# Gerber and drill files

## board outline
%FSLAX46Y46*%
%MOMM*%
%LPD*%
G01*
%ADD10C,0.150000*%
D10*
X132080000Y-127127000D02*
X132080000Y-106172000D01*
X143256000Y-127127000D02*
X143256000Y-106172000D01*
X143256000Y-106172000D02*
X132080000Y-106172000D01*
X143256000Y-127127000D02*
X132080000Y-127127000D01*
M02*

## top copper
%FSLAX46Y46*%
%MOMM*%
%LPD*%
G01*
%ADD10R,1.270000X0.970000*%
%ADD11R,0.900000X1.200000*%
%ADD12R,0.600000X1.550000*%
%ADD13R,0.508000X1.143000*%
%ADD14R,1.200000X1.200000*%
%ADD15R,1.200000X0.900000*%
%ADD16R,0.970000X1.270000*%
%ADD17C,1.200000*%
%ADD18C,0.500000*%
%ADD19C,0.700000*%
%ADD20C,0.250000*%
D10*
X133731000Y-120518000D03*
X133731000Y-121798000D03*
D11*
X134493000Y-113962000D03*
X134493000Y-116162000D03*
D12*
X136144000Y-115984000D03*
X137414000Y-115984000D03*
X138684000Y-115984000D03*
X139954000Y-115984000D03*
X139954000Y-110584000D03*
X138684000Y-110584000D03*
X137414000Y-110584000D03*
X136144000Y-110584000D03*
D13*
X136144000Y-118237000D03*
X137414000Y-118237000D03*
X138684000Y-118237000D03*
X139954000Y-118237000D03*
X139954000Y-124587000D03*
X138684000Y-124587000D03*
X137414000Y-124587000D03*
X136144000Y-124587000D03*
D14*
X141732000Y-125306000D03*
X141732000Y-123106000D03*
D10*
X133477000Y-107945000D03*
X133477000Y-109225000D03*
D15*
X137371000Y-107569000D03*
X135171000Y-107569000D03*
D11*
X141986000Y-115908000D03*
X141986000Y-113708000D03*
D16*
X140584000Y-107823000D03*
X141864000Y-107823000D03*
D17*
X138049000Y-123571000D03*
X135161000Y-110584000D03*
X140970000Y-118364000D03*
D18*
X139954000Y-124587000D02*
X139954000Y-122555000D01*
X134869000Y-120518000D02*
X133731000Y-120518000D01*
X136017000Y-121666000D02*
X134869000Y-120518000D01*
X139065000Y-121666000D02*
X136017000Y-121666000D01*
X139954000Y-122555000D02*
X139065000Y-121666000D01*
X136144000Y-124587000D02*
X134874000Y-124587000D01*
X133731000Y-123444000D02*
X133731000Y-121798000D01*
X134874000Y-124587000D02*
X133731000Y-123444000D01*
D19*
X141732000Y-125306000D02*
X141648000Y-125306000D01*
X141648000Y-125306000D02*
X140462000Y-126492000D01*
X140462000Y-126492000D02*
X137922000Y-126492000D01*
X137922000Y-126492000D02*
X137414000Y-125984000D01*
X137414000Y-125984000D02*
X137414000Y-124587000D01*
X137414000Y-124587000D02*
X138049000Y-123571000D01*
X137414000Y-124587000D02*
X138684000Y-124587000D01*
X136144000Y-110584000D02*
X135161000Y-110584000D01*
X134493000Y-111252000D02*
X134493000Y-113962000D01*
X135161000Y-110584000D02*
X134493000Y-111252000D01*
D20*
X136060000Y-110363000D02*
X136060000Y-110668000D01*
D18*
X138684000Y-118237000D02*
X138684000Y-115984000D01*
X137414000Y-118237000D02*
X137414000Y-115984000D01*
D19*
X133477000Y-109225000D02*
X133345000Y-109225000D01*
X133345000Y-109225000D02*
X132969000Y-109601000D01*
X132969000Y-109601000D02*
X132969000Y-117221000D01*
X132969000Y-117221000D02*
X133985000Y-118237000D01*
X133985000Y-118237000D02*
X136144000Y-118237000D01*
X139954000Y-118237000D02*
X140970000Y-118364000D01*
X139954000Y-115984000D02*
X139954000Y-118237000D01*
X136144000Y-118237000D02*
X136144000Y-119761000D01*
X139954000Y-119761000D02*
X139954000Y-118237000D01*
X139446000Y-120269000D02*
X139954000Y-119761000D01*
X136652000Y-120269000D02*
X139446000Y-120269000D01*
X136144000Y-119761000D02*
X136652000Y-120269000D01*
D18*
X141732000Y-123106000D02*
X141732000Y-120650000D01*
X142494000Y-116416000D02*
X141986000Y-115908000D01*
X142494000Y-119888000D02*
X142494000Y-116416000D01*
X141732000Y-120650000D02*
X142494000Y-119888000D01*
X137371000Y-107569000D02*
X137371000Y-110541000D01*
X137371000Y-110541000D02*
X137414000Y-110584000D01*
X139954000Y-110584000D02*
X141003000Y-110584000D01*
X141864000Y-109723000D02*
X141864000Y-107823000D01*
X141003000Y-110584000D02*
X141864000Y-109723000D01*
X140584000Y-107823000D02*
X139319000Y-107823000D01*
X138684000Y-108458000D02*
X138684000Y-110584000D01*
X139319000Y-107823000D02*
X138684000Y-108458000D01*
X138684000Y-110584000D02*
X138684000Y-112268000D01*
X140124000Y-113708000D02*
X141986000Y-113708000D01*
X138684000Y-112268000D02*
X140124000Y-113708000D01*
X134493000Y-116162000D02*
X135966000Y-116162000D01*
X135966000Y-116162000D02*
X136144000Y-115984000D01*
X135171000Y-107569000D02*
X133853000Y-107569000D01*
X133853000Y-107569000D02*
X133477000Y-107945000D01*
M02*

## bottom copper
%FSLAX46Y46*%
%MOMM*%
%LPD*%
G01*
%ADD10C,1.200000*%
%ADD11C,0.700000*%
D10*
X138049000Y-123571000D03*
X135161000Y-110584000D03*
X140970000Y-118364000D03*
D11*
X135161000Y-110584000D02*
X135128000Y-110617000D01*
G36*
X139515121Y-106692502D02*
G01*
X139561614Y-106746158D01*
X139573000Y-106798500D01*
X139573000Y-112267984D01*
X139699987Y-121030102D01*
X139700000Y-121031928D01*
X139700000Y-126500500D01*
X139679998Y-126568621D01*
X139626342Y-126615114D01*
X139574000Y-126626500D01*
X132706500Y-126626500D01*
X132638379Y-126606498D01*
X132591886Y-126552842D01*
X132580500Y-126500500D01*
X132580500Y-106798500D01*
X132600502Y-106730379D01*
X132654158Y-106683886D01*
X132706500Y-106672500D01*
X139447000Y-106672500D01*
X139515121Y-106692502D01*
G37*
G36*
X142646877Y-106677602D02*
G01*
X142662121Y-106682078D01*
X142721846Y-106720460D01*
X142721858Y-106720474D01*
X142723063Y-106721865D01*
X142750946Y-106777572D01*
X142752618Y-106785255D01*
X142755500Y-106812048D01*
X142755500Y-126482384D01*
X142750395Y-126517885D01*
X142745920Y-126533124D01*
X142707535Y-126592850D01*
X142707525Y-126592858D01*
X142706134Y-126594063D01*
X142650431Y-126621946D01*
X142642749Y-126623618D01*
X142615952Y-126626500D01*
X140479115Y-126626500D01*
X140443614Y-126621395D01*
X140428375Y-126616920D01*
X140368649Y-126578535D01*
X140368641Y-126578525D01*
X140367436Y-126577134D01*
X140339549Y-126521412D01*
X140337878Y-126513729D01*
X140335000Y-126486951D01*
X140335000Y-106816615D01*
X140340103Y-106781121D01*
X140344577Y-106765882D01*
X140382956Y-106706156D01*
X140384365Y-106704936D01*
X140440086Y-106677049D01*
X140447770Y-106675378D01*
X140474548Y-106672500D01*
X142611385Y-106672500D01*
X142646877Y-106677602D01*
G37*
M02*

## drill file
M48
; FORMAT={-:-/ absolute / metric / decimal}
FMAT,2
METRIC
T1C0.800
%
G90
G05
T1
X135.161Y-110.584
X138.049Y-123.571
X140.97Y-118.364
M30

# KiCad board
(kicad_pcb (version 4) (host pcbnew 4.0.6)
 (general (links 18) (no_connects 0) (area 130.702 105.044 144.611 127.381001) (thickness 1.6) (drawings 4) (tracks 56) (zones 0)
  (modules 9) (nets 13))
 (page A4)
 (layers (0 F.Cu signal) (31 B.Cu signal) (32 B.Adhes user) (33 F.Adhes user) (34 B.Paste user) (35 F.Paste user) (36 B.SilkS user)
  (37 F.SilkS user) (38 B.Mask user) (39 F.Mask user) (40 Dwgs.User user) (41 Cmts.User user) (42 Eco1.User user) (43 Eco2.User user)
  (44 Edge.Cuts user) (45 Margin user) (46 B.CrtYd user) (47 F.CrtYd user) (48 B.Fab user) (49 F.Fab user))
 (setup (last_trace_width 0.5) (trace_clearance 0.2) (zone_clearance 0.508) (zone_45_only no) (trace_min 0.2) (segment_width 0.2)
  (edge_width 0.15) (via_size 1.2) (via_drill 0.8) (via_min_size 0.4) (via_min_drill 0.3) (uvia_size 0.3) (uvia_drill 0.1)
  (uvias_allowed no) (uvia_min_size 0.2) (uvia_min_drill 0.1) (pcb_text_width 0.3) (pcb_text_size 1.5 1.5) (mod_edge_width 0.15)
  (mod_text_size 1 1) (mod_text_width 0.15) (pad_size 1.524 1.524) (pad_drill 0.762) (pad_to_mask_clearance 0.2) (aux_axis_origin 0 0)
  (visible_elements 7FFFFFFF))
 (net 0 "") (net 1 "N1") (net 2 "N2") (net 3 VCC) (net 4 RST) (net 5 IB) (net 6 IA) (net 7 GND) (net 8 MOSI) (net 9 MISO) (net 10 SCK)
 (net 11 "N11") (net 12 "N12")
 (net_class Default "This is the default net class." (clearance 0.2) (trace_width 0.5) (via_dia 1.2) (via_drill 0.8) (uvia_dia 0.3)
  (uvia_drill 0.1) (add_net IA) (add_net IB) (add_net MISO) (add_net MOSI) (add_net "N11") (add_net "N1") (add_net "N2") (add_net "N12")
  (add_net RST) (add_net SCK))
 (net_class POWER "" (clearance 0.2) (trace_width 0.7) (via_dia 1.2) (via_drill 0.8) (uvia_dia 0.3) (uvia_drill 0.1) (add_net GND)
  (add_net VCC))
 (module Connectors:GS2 (layer F.Cu) (at 133.731 121.158)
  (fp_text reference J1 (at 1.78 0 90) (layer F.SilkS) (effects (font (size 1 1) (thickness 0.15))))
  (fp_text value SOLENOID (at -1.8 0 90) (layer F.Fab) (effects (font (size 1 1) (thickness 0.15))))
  (pad 1 smd rect (at 0 -0.64) (size 1.27 0.97) (layers F.Cu F.Paste F.Mask) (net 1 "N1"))
  (pad 2 smd rect (at 0 0.64) (size 1.27 0.97) (layers F.Cu F.Paste F.Mask) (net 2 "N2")))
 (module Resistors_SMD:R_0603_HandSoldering (layer F.Cu) (at 134.493 115.062 270)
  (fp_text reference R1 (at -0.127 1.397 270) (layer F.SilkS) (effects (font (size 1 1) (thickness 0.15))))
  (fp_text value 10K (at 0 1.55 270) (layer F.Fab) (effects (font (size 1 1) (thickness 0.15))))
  (pad 1 smd rect (at -1.1 0 270) (size 1.2 0.9) (layers F.Cu F.Paste F.Mask) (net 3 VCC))
  (pad 2 smd rect (at 1.1 0 270) (size 1.2 0.9) (layers F.Cu F.Paste F.Mask) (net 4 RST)))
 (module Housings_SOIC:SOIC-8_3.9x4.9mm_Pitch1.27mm (layer F.Cu) (at 138.049 113.284 90)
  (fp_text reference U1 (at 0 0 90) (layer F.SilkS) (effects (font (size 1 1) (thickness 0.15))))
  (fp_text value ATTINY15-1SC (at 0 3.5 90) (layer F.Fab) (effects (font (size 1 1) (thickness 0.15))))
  (pad 1 smd rect (at -2.7 -1.905 90) (size 1.55 0.6) (layers F.Cu F.Paste F.Mask) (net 4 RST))
  (pad 2 smd rect (at -2.7 -0.635 90) (size 1.55 0.6) (layers F.Cu F.Paste F.Mask) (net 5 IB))
  (pad 3 smd rect (at -2.7 0.635 90) (size 1.55 0.6) (layers F.Cu F.Paste F.Mask) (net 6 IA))
  (pad 4 smd rect (at -2.7 1.905 90) (size 1.55 0.6) (layers F.Cu F.Paste F.Mask) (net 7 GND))
  (pad 5 smd rect (at 2.7 1.905 90) (size 1.55 0.6) (layers F.Cu F.Paste F.Mask) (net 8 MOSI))
  (pad 6 smd rect (at 2.7 0.635 90) (size 1.55 0.6) (layers F.Cu F.Paste F.Mask) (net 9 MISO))
  (pad 7 smd rect (at 2.7 -0.635 90) (size 1.55 0.6) (layers F.Cu F.Paste F.Mask) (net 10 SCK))
  (pad 8 smd rect (at 2.7 -1.905 90) (size 1.55 0.6) (layers F.Cu F.Paste F.Mask) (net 3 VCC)))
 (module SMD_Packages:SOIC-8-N (layer F.Cu) (at 138.049 121.412)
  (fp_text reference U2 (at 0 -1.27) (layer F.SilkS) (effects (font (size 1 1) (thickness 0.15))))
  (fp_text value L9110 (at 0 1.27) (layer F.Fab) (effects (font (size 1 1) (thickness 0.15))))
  (pad 8 smd rect (at -1.905 -3.175) (size 0.508 1.143) (layers F.Cu F.Paste F.Mask) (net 7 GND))
  (pad 7 smd rect (at -0.635 -3.175) (size 0.508 1.143) (layers F.Cu F.Paste F.Mask) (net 5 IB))
  (pad 6 smd rect (at 0.635 -3.175) (size 0.508 1.143) (layers F.Cu F.Paste F.Mask) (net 6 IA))
  (pad 5 smd rect (at 1.905 -3.175) (size 0.508 1.143) (layers F.Cu F.Paste F.Mask) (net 7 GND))
  (pad 4 smd rect (at 1.905 3.175) (size 0.508 1.143) (layers F.Cu F.Paste F.Mask) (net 1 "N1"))
  (pad 3 smd rect (at 0.635 3.175) (size 0.508 1.143) (layers F.Cu F.Paste F.Mask) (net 3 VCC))
  (pad 2 smd rect (at -0.635 3.175) (size 0.508 1.143) (layers F.Cu F.Paste F.Mask) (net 3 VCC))
  (pad 1 smd rect (at -1.905 3.175) (size 0.508 1.143) (layers F.Cu F.Paste F.Mask) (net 2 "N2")))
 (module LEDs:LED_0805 (layer F.Cu) (at 141.732 124.206 270)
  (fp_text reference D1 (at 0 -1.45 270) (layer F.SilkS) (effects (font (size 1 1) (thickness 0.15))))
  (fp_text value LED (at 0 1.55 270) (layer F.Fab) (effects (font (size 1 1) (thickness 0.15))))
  (pad 2 smd rect (at 1.1 0 90) (size 1.2 1.2) (layers F.Cu F.Paste F.Mask) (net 3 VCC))
  (pad 1 smd rect (at -1.1 0 90) (size 1.2 1.2) (layers F.Cu F.Paste F.Mask) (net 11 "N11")))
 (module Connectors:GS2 (layer F.Cu) (at 133.477 108.585)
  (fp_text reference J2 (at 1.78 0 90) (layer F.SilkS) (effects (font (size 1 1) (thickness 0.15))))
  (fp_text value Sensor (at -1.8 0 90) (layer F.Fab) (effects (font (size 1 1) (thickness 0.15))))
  (pad 1 smd rect (at 0 -0.64) (size 1.27 0.97) (layers F.Cu F.Paste F.Mask) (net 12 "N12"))
  (pad 2 smd rect (at 0 0.64) (size 1.27 0.97) (layers F.Cu F.Paste F.Mask) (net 7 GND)))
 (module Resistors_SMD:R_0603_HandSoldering (layer F.Cu) (at 136.271 107.569 180)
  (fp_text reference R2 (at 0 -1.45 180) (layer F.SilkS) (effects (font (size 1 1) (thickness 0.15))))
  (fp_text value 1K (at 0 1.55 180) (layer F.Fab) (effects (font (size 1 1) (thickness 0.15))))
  (pad 1 smd rect (at -1.1 0 180) (size 1.2 0.9) (layers F.Cu F.Paste F.Mask) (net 10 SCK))
  (pad 2 smd rect (at 1.1 0 180) (size 1.2 0.9) (layers F.Cu F.Paste F.Mask) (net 12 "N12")))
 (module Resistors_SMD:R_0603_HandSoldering (layer F.Cu) (at 141.986 114.808 90)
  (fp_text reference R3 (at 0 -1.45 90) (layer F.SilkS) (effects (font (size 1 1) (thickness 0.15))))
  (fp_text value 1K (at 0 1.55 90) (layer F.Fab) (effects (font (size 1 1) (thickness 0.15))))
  (pad 1 smd rect (at -1.1 0 90) (size 1.2 0.9) (layers F.Cu F.Paste F.Mask) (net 11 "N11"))
  (pad 2 smd rect (at 1.1 0 90) (size 1.2 0.9) (layers F.Cu F.Paste F.Mask) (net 9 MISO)))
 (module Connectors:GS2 (layer F.Cu) (at 141.224 107.823 90)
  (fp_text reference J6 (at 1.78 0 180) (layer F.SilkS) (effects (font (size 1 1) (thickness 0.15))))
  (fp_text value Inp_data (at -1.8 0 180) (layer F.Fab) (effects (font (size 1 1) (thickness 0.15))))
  (pad 1 smd rect (at 0 -0.64 90) (size 1.27 0.97) (layers F.Cu F.Paste F.Mask) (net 9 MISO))
  (pad 2 smd rect (at 0 0.64 90) (size 1.27 0.97) (layers F.Cu F.Paste F.Mask) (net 8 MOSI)))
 (gr_line (start 132.08 127.127) (end 132.08 106.172) (angle 90) (layer Edge.Cuts) (width 0.15))
 (gr_line (start 143.256 127.127) (end 143.256 106.172) (angle 90) (layer Edge.Cuts) (width 0.15))
 (gr_line (start 143.256 106.172) (end 132.08 106.172) (angle 90) (layer Edge.Cuts) (width 0.15))
 (gr_line (start 143.256 127.127) (end 132.08 127.127) (angle 90) (layer Edge.Cuts) (width 0.15))
 (segment (start 139.954 124.587) (end 139.954 122.555) (width 0.5) (layer F.Cu) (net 1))
 (segment (start 134.869 120.518) (end 133.731 120.518) (width 0.5) (layer F.Cu) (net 1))
 (segment (start 136.017 121.666) (end 134.869 120.518) (width 0.5) (layer F.Cu) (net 1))
 (segment (start 139.065 121.666) (end 136.017 121.666) (width 0.5) (layer F.Cu) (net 1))
 (segment (start 139.954 122.555) (end 139.065 121.666) (width 0.5) (layer F.Cu) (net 1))
 (segment (start 136.144 124.587) (end 134.874 124.587) (width 0.5) (layer F.Cu) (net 2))
 (segment (start 133.731 123.444) (end 133.731 121.798) (width 0.5) (layer F.Cu) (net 2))
 (segment (start 134.874 124.587) (end 133.731 123.444) (width 0.5) (layer F.Cu) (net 2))
 (segment (start 141.732 125.306) (end 141.648 125.306) (width 0.7) (layer F.Cu) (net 3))
 (segment (start 141.648 125.306) (end 140.462 126.492) (width 0.7) (layer F.Cu) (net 3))
 (segment (start 140.462 126.492) (end 137.922 126.492) (width 0.7) (layer F.Cu) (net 3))
 (segment (start 137.922 126.492) (end 137.414 125.984) (width 0.7) (layer F.Cu) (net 3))
 (segment (start 137.414 125.984) (end 137.414 124.587) (width 0.7) (layer F.Cu) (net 3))
 (segment (start 137.414 124.587) (end 138.049 123.571) (width 0.7) (layer F.Cu) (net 3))
 (via (at 138.049 123.571) (size 1.2) (drill 0.8) (layers F.Cu B.Cu) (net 3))
 (segment (start 137.414 124.587) (end 138.684 124.587) (width 0.7) (layer F.Cu) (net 3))
 (segment (start 136.144 110.584) (end 135.161 110.584) (width 0.7) (layer F.Cu) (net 3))
 (via (at 135.161 110.584) (size 1.2) (drill 0.8) (layers F.Cu B.Cu) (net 3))
 (segment (start 135.161 110.584) (end 135.128 110.617) (width 0.7) (layer B.Cu) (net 3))
 (segment (start 134.493 111.252) (end 134.493 113.962) (width 0.7) (layer F.Cu) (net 3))
 (segment (start 135.161 110.584) (end 134.493 111.252) (width 0.7) (layer F.Cu) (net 3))
 (segment (start 136.06 110.363) (end 136.06 110.668) (width 0.25) (layer F.Cu) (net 3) (status 30))
 (segment (start 138.684 118.237) (end 138.684 115.984) (width 0.5) (layer F.Cu) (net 6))
 (segment (start 137.414 118.237) (end 137.414 115.984) (width 0.5) (layer F.Cu) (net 5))
 (segment (start 133.477 109.225) (end 133.345 109.225) (width 0.7) (layer F.Cu) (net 7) (status C00000))
 (segment (start 133.345 109.225) (end 132.969 109.601) (width 0.7) (layer F.Cu) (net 7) (status C00000))
 (segment (start 132.969 109.601) (end 132.969 117.221) (width 0.7) (layer F.Cu) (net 7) (status 400000))
 (segment (start 132.969 117.221) (end 133.985 118.237) (width 0.7) (layer F.Cu) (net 7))
 (segment (start 133.985 118.237) (end 136.144 118.237) (width 0.7) (layer F.Cu) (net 7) (status 800000))
 (segment (start 139.954 118.237) (end 140.97 118.364) (width 0.7) (layer F.Cu) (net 7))
 (via (at 140.97 118.364) (size 1.2) (drill 0.8) (layers F.Cu B.Cu) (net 7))
 (segment (start 139.954 115.984) (end 139.954 118.237) (width 0.7) (layer F.Cu) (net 7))
 (segment (start 136.144 118.237) (end 136.144 119.761) (width 0.7) (layer F.Cu) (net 7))
 (segment (start 139.954 119.761) (end 139.954 118.237) (width 0.7) (layer F.Cu) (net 7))
 (segment (start 139.446 120.269) (end 139.954 119.761) (width 0.7) (layer F.Cu) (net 7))
 (segment (start 136.652 120.269) (end 139.446 120.269) (width 0.7) (layer F.Cu) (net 7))
 (segment (start 136.144 119.761) (end 136.652 120.269) (width 0.7) (layer F.Cu) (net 7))
 (segment (start 141.732 123.106) (end 141.732 120.65) (width 0.5) (layer F.Cu) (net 11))
 (segment (start 142.494 116.416) (end 141.986 115.908) (width 0.5) (layer F.Cu) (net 11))
 (segment (start 142.494 119.888) (end 142.494 116.416) (width 0.5) (layer F.Cu) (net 11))
 (segment (start 141.732 120.65) (end 142.494 119.888) (width 0.5) (layer F.Cu) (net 11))
 (segment (start 137.371 107.569) (end 137.371 110.541) (width 0.5) (layer F.Cu) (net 10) (status C00000))
 (segment (start 137.371 110.541) (end 137.414 110.584) (width 0.5) (layer F.Cu) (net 10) (status C00000))
 (segment (start 139.954 110.584) (end 141.003 110.584) (width 0.5) (layer F.Cu) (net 8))
 (segment (start 141.864 109.723) (end 141.864 107.823) (width 0.5) (layer F.Cu) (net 8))
 (segment (start 141.003 110.584) (end 141.864 109.723) (width 0.5) (layer F.Cu) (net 8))
 (segment (start 140.584 107.823) (end 139.319 107.823) (width 0.5) (layer F.Cu) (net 9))
 (segment (start 138.684 108.458) (end 138.684 110.584) (width 0.5) (layer F.Cu) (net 9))
 (segment (start 139.319 107.823) (end 138.684 108.458) (width 0.5) (layer F.Cu) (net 9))
 (segment (start 138.684 110.584) (end 138.684 112.268) (width 0.5) (layer F.Cu) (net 9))
 (segment (start 140.124 113.708) (end 141.986 113.708) (width 0.5) (layer F.Cu) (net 9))
 (segment (start 138.684 112.268) (end 140.124 113.708) (width 0.5) (layer F.Cu) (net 9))
 (segment (start 134.493 116.162) (end 135.966 116.162) (width 0.5) (layer F.Cu) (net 4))
 (segment (start 135.966 116.162) (end 136.144 115.984) (width 0.5) (layer F.Cu) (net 4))
 (segment (start 135.171 107.569) (end 133.853 107.569) (width 0.5) (layer F.Cu) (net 12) (status C00000))
 (segment (start 133.853 107.569) (end 133.477 107.945) (width 0.5) (layer F.Cu) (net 12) (status C00000))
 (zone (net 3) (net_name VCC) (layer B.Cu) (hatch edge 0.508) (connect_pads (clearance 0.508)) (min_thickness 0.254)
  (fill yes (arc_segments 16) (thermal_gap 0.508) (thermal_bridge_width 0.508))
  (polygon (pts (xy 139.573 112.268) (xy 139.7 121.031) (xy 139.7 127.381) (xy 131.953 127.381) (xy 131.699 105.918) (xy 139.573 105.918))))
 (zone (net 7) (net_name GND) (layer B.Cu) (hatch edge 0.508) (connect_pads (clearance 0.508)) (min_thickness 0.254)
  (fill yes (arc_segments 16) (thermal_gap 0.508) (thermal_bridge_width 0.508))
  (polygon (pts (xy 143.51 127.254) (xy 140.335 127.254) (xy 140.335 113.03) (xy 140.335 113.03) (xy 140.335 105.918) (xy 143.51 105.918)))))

